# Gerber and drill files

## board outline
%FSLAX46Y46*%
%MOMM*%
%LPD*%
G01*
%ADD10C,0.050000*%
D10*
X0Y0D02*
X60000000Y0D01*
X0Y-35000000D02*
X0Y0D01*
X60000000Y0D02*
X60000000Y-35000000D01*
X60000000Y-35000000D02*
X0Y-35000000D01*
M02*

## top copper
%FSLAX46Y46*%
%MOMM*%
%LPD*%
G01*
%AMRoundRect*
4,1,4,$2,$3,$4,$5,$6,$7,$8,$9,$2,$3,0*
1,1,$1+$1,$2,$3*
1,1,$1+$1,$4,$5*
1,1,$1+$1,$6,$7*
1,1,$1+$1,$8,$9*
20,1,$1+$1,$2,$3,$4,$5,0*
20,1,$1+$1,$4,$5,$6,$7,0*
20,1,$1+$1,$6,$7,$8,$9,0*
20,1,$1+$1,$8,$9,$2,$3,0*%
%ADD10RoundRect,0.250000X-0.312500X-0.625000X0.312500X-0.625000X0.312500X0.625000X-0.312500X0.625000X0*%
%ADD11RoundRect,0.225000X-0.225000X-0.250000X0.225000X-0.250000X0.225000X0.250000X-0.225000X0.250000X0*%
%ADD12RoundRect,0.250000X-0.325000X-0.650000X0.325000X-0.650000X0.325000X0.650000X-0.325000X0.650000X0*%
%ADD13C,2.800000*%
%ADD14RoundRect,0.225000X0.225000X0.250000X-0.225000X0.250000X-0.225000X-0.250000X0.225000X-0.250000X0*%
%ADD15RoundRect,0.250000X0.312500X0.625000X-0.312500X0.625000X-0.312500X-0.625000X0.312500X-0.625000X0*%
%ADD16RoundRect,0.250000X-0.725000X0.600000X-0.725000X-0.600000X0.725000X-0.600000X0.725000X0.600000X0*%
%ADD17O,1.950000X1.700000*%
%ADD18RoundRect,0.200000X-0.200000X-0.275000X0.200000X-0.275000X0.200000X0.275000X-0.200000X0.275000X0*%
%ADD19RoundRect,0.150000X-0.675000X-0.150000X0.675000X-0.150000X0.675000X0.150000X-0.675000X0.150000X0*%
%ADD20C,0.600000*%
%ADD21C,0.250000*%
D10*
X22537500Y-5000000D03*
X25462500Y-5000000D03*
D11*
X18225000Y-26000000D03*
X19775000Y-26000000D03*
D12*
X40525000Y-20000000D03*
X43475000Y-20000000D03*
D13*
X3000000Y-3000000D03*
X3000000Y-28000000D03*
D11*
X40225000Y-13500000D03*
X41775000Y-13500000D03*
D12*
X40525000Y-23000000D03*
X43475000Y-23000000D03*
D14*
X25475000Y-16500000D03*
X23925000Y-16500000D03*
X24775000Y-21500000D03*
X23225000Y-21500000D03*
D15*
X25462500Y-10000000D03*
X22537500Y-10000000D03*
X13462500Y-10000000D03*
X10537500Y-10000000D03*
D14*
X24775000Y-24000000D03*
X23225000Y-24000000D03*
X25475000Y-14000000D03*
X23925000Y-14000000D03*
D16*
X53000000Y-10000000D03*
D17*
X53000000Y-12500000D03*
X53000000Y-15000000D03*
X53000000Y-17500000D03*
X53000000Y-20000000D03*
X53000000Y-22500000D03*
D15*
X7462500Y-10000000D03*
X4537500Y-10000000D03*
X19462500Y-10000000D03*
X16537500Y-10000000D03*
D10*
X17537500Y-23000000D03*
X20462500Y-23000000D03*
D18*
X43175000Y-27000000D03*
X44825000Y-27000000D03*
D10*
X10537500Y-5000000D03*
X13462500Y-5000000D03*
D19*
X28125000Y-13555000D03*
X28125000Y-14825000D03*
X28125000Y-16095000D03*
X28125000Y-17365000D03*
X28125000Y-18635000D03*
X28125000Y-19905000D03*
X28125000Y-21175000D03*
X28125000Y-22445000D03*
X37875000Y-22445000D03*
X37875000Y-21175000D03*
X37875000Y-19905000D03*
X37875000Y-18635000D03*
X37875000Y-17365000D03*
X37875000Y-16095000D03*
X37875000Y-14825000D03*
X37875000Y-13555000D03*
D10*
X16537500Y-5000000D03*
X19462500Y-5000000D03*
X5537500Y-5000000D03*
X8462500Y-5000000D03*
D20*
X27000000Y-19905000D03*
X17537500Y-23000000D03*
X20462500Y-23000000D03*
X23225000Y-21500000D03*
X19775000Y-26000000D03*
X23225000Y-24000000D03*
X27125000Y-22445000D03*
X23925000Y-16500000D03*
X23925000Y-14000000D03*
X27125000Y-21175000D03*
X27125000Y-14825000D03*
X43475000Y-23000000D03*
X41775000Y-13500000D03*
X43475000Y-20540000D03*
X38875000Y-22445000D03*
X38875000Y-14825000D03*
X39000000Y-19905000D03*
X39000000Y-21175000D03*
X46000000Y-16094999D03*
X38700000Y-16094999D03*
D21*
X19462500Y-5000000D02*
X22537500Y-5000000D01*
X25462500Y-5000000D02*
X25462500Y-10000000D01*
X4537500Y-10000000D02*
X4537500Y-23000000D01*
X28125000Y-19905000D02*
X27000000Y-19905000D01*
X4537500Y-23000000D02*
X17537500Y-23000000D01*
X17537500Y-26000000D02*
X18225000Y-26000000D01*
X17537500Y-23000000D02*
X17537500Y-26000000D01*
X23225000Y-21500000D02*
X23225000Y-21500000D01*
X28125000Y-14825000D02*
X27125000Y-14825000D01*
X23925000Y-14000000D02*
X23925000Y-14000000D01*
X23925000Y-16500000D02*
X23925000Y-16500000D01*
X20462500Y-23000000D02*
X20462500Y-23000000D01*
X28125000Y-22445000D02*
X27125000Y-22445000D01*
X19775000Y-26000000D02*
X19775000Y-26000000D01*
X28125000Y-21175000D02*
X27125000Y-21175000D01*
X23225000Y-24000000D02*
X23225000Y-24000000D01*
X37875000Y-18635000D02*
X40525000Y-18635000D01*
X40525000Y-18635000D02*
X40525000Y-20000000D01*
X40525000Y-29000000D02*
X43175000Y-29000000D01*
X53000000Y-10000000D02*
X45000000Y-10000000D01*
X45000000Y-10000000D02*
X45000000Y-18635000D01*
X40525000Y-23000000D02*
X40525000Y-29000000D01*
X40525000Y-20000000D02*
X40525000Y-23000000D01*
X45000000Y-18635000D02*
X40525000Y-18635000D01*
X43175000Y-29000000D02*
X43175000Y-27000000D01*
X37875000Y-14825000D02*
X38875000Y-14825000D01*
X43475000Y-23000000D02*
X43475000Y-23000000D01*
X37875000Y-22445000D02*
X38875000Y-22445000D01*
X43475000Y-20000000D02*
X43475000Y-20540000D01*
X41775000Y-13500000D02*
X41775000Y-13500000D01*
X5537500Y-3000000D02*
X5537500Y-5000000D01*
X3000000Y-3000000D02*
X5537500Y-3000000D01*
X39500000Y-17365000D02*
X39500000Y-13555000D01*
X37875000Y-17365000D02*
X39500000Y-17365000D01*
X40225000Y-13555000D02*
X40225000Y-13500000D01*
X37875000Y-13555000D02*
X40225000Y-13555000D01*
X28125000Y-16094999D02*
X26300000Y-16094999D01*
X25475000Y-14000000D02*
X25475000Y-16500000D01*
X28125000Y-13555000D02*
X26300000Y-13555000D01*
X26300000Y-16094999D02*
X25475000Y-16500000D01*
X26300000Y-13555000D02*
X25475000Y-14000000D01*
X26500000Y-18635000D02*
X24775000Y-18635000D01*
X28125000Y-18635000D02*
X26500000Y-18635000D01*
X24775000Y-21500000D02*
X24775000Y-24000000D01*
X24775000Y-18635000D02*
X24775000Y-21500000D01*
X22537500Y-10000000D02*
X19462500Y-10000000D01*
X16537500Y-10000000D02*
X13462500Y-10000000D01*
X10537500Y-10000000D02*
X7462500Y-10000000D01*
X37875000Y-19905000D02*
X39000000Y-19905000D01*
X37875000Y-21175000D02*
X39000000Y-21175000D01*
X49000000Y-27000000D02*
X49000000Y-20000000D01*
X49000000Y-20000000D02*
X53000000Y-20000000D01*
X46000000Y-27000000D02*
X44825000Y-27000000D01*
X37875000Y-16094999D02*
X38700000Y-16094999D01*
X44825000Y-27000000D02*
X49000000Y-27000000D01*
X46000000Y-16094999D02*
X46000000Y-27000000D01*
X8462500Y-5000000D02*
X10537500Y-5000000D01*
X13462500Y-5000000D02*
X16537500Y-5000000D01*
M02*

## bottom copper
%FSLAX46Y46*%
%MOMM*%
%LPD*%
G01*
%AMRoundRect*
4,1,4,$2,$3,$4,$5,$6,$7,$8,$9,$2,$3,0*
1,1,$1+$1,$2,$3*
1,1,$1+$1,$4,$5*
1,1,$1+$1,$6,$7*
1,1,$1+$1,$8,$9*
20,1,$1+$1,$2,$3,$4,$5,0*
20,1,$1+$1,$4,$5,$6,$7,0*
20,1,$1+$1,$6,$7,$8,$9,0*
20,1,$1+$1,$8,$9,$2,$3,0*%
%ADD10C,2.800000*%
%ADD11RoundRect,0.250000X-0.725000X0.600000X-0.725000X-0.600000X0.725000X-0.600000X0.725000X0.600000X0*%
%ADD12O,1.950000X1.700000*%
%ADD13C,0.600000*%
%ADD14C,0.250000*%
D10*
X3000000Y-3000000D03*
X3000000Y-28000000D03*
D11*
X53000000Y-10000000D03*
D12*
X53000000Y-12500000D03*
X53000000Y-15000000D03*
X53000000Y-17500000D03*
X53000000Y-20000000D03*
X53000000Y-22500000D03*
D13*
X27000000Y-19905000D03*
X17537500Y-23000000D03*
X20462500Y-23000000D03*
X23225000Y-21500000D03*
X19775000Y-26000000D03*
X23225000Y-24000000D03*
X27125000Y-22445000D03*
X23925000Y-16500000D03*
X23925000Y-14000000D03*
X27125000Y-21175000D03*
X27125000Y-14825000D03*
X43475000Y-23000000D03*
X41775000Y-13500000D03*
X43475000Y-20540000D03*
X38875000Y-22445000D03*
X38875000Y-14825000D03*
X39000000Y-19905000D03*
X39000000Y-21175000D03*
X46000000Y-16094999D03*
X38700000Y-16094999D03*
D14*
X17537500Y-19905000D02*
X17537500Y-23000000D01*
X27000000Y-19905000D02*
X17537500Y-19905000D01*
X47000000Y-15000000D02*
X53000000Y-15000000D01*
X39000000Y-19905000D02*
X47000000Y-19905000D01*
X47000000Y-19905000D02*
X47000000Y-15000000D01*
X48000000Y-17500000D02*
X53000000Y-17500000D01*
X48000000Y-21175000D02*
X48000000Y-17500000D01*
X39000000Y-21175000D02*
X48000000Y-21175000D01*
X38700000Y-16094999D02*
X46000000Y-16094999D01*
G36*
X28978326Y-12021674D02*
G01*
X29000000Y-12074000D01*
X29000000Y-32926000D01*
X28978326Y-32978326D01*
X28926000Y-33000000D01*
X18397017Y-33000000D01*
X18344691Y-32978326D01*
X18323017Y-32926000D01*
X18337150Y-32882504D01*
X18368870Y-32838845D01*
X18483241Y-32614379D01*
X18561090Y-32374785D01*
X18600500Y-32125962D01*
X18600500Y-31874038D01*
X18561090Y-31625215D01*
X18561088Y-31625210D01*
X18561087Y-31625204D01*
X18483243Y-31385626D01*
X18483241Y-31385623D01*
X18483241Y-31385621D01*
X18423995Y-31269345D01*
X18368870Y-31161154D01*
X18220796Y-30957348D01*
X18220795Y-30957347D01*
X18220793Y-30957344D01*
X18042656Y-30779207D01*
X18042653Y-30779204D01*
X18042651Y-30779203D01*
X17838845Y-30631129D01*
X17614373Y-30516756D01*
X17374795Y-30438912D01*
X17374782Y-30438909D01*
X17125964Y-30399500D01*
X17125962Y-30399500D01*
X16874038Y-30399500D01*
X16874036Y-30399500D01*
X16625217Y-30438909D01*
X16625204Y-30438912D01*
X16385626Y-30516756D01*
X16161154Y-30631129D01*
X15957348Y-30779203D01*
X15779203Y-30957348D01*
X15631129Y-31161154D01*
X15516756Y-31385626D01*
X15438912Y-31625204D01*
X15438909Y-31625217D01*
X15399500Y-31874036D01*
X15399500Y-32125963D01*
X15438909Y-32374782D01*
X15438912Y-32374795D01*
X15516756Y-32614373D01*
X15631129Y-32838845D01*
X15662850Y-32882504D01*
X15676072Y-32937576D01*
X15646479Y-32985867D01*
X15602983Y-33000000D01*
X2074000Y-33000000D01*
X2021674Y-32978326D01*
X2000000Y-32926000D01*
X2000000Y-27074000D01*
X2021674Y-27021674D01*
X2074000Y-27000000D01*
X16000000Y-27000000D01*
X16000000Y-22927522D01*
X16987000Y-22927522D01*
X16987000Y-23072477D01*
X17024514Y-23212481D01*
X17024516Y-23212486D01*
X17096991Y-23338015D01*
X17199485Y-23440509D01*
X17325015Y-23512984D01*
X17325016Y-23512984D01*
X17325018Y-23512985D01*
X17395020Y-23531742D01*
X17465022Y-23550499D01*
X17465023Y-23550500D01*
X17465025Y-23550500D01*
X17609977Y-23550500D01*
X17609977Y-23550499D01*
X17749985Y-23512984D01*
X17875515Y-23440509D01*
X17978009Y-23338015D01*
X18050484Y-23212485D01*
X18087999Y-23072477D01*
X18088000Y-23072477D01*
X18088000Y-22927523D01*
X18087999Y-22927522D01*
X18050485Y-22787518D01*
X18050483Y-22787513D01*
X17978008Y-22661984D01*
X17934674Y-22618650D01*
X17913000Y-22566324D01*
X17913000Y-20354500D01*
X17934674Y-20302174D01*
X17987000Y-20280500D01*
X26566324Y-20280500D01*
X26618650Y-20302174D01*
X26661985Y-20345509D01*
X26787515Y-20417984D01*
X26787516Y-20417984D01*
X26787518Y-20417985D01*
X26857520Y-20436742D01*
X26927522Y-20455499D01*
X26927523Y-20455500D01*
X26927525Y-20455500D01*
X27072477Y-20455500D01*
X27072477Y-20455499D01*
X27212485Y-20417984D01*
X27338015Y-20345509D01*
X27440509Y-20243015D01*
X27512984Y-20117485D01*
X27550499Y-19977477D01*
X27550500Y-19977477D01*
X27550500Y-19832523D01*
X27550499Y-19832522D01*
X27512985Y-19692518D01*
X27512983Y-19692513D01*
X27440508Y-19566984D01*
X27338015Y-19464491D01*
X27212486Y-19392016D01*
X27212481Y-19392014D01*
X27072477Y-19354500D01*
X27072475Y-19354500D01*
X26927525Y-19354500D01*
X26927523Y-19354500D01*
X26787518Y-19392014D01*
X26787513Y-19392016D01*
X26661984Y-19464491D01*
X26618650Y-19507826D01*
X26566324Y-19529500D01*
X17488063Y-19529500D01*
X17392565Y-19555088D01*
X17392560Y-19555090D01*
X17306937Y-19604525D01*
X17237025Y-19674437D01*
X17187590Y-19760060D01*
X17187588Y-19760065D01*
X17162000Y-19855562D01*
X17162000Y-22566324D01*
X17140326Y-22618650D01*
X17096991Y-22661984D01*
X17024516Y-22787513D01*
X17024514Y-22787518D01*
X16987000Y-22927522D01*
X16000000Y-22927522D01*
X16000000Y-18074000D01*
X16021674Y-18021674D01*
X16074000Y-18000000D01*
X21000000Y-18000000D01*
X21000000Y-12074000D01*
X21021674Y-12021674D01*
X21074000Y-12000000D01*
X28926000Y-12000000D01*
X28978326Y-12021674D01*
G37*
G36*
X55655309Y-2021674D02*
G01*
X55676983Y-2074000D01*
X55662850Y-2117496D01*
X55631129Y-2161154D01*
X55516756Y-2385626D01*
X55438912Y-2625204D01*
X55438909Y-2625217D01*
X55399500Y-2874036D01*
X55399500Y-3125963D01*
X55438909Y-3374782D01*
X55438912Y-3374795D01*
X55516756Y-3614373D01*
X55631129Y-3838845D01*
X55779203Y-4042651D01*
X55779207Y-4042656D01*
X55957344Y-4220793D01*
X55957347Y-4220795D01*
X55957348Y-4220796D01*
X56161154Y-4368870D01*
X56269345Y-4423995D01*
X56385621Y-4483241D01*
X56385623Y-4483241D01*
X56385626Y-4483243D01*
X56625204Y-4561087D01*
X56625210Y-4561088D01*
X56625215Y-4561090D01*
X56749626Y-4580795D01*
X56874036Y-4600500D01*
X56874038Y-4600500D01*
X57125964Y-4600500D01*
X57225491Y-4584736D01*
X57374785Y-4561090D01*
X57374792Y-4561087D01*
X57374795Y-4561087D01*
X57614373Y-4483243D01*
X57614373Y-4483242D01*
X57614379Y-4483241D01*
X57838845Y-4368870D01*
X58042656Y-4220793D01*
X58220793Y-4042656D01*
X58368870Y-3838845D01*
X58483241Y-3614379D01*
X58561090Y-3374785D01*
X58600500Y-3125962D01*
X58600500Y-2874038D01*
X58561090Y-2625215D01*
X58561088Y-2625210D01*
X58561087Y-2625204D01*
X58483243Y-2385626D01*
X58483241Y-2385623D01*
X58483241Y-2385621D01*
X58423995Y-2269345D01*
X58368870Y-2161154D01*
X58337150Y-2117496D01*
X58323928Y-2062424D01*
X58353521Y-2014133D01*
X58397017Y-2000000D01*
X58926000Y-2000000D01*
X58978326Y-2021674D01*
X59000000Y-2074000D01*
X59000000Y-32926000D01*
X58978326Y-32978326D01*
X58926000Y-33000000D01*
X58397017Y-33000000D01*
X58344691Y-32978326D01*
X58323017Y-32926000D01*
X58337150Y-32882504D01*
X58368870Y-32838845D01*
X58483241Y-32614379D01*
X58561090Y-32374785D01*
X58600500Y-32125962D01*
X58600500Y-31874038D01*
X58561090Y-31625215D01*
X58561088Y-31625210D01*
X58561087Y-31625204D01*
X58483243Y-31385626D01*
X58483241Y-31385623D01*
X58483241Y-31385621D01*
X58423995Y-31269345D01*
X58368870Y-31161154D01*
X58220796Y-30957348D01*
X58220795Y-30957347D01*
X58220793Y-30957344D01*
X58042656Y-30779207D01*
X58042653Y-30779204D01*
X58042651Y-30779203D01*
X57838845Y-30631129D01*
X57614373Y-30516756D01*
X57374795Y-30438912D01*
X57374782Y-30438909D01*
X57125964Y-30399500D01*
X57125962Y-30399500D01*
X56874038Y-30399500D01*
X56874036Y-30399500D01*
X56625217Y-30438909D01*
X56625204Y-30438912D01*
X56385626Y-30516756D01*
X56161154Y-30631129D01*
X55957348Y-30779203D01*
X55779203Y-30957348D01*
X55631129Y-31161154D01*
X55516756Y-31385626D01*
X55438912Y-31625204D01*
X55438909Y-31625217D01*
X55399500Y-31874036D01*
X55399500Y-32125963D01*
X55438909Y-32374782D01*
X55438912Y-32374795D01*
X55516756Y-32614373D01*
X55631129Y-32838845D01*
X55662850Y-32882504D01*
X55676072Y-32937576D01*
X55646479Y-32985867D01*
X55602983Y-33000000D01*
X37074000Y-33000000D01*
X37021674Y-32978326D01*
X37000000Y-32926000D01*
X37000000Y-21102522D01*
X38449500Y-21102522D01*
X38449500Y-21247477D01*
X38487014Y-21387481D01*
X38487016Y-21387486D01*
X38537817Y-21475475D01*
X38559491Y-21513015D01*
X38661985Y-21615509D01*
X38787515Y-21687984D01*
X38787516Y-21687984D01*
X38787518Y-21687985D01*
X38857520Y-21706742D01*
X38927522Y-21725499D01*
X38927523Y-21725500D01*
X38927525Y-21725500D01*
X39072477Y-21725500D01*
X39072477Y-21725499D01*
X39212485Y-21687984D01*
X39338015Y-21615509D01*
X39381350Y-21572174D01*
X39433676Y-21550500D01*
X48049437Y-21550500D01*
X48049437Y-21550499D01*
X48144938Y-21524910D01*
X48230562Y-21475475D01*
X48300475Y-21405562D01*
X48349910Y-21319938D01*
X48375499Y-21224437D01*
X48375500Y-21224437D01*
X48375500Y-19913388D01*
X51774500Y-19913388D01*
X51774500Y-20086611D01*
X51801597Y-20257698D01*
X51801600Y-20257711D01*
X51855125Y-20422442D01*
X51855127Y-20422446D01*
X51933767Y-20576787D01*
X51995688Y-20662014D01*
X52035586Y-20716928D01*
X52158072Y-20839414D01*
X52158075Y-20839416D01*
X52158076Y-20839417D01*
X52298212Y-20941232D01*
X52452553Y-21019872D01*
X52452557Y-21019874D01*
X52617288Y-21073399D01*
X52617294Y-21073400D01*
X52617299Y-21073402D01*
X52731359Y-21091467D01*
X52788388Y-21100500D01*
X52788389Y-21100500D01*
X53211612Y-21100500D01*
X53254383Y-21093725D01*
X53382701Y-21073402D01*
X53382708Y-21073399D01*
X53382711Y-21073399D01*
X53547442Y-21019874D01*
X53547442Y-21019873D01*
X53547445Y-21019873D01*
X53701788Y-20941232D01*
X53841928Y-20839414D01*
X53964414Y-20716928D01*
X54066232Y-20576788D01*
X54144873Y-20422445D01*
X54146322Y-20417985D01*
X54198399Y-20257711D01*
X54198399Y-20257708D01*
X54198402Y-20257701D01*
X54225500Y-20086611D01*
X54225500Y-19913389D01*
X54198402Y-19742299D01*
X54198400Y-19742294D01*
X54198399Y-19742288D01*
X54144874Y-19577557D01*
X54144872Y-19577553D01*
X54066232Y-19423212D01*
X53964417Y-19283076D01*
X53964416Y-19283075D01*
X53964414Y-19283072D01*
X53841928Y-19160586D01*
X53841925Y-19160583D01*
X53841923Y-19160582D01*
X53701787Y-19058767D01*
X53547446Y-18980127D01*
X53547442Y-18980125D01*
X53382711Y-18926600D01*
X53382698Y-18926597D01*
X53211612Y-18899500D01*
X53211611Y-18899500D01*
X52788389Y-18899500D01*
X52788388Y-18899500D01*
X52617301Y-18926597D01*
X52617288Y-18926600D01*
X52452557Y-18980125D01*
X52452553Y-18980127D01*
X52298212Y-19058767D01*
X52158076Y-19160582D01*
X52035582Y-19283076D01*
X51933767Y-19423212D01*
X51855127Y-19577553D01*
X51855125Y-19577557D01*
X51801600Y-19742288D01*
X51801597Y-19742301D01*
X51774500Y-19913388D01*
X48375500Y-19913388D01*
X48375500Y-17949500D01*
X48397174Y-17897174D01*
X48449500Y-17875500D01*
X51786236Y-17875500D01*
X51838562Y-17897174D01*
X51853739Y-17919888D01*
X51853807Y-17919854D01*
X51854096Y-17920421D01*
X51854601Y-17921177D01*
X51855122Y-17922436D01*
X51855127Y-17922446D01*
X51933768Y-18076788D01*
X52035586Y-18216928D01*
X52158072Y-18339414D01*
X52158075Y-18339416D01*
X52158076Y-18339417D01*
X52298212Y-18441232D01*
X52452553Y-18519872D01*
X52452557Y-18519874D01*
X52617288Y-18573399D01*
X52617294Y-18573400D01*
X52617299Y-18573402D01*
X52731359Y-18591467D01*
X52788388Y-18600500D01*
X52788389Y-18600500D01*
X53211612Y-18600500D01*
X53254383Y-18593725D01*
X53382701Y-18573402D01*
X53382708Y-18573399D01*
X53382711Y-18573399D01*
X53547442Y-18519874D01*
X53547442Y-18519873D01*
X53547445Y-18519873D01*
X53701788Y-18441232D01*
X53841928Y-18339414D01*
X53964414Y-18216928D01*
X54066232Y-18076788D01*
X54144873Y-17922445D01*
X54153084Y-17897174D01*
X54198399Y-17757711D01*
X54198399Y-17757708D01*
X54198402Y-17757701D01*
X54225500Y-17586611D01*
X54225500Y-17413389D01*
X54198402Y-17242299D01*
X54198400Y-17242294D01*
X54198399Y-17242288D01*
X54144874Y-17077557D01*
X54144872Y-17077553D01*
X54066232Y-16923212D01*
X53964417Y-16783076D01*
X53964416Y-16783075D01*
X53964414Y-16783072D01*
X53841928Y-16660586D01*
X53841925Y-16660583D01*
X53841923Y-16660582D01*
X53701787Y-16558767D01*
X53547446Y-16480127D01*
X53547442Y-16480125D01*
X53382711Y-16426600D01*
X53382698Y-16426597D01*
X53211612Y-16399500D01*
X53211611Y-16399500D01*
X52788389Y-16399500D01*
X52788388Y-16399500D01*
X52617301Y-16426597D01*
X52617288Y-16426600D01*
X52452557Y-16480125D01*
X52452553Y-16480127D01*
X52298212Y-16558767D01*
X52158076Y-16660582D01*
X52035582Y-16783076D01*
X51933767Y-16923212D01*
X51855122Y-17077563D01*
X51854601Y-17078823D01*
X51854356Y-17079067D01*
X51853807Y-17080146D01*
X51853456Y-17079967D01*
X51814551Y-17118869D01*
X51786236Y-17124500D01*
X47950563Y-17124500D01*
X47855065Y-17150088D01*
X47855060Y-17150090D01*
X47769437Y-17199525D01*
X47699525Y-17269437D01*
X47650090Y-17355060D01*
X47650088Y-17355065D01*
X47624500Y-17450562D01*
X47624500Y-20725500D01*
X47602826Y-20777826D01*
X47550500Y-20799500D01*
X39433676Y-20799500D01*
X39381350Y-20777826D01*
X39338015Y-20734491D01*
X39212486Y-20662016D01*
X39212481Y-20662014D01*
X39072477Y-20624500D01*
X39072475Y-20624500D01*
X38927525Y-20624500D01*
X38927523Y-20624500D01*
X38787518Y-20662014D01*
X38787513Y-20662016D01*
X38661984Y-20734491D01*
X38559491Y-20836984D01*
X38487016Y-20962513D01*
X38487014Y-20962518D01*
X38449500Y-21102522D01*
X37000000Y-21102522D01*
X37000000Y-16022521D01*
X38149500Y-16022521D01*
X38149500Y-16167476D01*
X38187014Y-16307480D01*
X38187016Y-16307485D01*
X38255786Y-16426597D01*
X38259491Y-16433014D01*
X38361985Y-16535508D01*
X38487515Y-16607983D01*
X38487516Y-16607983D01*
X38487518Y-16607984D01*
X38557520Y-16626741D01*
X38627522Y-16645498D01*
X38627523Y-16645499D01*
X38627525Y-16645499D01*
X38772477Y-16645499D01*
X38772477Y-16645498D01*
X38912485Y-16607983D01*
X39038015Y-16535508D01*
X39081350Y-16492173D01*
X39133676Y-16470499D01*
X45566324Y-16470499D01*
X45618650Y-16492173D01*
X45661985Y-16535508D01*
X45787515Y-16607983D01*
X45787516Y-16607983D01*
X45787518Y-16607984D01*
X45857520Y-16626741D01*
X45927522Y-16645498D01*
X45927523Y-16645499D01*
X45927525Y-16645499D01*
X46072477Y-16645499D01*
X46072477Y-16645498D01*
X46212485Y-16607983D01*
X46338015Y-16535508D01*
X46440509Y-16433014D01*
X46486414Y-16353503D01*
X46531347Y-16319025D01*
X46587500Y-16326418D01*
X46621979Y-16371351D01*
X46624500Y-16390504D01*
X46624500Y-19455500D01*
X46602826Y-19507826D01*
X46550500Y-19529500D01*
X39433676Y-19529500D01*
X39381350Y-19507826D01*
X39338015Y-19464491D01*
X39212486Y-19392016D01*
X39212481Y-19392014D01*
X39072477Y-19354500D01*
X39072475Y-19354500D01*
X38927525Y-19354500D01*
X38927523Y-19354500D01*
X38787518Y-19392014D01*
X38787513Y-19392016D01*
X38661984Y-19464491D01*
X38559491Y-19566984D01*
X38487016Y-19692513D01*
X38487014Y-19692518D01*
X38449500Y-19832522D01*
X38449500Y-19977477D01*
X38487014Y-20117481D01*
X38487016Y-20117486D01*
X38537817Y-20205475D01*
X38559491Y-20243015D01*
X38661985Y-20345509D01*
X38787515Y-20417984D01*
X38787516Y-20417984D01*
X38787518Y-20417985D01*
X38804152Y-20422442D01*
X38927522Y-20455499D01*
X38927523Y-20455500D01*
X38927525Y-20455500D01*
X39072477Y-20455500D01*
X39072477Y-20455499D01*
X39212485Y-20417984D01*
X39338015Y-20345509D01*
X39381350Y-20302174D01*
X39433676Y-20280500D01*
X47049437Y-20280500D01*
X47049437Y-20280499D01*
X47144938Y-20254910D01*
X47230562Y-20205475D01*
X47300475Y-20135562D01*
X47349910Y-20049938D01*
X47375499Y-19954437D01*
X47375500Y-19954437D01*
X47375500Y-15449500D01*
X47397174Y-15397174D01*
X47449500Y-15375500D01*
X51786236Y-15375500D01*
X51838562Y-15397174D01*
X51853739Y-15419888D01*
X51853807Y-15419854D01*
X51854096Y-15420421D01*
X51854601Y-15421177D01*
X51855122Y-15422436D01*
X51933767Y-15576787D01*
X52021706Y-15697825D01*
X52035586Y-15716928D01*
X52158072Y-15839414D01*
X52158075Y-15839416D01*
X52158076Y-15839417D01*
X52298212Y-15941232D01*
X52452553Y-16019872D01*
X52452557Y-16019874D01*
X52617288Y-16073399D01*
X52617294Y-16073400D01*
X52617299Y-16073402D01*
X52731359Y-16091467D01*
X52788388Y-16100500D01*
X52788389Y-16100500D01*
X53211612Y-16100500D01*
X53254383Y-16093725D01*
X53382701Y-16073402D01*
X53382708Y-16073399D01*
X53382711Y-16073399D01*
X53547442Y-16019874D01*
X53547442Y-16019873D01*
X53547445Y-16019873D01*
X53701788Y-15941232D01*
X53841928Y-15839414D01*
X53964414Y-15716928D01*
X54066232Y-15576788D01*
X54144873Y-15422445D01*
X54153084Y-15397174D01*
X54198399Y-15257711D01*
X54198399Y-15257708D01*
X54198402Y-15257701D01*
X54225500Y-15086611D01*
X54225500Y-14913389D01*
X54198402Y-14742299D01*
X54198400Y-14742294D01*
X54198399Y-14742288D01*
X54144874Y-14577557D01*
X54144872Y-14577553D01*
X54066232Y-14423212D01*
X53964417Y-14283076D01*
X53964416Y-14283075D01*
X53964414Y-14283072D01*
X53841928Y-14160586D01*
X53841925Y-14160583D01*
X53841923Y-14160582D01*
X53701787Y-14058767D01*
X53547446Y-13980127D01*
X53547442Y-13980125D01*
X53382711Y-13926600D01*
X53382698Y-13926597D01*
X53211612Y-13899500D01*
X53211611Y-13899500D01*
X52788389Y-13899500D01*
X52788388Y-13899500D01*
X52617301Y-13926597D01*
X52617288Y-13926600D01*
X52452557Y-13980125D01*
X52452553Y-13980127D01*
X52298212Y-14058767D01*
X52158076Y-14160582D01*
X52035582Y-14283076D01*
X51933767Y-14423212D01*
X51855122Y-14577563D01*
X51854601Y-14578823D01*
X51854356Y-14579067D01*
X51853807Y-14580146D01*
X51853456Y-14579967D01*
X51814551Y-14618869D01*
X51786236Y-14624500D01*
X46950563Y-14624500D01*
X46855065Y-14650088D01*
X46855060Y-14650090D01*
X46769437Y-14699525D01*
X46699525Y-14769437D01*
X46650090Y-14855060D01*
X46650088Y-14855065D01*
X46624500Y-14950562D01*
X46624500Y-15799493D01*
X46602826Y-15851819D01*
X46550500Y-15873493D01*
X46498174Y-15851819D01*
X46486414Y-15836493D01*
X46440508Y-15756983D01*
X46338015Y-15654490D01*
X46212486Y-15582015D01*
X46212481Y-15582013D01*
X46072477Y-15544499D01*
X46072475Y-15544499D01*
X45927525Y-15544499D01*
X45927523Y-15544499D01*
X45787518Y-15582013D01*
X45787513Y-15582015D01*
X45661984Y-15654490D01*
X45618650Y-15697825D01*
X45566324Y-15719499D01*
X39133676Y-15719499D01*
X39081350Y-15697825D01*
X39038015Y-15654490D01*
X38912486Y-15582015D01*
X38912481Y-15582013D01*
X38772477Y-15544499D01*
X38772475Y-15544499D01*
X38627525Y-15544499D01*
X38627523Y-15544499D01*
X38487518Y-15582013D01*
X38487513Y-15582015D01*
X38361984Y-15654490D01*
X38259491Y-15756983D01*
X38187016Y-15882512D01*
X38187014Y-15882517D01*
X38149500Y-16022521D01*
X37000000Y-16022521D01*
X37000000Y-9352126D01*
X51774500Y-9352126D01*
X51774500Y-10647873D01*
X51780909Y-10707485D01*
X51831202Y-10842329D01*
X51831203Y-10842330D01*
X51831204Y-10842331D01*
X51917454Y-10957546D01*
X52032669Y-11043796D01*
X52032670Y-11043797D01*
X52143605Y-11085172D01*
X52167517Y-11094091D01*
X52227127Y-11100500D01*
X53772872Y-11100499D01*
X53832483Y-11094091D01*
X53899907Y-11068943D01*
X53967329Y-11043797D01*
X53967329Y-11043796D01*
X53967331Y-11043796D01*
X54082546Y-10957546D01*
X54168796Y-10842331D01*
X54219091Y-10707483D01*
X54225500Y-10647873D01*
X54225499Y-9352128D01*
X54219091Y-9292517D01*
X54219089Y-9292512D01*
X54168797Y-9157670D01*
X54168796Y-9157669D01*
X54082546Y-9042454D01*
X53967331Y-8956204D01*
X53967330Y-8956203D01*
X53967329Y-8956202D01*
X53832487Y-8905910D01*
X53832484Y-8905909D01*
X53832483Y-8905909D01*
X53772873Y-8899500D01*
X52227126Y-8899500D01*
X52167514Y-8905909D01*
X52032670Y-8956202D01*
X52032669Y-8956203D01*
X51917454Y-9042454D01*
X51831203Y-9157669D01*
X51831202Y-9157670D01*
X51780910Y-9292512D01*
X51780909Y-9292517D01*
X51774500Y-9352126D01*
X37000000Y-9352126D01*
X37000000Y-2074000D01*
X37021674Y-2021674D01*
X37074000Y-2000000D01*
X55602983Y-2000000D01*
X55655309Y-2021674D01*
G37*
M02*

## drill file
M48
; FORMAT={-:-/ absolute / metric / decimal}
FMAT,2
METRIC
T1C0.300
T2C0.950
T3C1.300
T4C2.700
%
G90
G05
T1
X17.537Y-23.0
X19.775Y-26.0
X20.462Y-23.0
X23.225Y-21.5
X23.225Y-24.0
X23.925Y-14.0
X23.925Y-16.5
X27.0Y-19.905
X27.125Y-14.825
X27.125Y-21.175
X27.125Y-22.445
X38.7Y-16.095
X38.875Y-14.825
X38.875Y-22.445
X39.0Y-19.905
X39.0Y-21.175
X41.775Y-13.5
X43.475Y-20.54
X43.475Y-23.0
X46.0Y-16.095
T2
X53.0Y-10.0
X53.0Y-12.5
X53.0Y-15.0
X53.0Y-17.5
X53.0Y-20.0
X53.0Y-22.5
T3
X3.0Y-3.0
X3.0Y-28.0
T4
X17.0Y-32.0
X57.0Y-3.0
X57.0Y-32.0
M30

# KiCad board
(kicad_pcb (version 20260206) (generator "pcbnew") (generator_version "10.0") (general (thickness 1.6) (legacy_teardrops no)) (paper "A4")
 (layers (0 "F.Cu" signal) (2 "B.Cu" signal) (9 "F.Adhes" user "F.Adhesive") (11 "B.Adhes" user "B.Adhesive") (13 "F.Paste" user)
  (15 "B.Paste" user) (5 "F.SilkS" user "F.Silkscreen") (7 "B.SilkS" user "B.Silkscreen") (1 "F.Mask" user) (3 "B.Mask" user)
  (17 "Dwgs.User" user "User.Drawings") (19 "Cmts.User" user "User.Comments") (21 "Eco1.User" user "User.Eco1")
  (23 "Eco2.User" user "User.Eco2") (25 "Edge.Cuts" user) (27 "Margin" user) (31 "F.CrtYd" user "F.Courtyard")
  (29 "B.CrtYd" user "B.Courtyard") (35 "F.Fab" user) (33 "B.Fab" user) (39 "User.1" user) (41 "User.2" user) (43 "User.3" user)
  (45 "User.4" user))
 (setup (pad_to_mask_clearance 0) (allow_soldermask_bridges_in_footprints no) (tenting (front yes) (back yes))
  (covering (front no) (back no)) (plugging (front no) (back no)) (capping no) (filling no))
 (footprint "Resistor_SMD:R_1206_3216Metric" (layer "F.Cu") (at 24 5)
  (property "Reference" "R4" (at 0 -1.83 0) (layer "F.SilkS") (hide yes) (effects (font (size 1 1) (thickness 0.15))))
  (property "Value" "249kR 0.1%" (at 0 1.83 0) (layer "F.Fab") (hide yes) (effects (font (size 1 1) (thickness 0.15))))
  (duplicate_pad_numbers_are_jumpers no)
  (pad "1" smd roundrect (at -1.4625 0) (size 1.125 1.75) (layers "F.Cu" "F.Mask" "F.Paste") (roundrect_rratio 0.222222) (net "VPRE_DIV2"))
  (pad "2" smd roundrect (at 1.4625 0) (size 1.125 1.75) (layers "F.Cu" "F.Mask" "F.Paste") (roundrect_rratio 0.222222) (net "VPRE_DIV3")))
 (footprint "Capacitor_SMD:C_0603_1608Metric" (layer "F.Cu") (at 19 26)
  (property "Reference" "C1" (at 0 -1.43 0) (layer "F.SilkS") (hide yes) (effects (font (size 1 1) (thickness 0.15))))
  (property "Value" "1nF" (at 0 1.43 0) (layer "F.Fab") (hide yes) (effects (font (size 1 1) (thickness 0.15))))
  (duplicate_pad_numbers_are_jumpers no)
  (pad "1" smd roundrect (at -0.775 0) (size 0.9 0.95) (layers "F.Cu" "F.Mask" "F.Paste") (roundrect_rratio 0.25) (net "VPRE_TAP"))
  (pad "2" smd roundrect (at 0.775 0) (size 0.9 0.95) (layers "F.Cu" "F.Mask" "F.Paste") (roundrect_rratio 0.25) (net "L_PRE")))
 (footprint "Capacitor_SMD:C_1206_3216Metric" (layer "F.Cu") (at 42 20)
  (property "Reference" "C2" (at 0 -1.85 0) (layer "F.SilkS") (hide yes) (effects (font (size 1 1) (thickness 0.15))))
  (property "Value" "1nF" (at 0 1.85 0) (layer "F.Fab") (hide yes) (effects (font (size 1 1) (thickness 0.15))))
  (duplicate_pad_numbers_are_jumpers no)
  (pad "1" smd roundrect (at -1.475 0) (size 1.15 1.8) (layers "F.Cu" "F.Mask" "F.Paste") (roundrect_rratio 0.217391) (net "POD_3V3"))
  (pad "2" smd roundrect (at 1.475 0) (size 1.15 1.8) (layers "F.Cu" "F.Mask" "F.Paste") (roundrect_rratio 0.217391) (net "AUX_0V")))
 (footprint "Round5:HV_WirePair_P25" (layer "F.Cu") (at 3 3)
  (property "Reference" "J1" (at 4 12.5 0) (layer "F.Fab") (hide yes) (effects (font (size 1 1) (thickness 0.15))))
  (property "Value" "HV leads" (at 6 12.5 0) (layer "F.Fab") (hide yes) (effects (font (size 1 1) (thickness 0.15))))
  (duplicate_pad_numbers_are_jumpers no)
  (pad "1" thru_hole circle (at 0 0) (size 2.8 2.8) (drill 1.3) (layers "*.Cu" "*.Mask") (remove_unused_layers no) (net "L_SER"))
  (pad "2" thru_hole circle (at 0 25) (size 2.8 2.8) (drill 1.3) (layers "*.Cu" "*.Mask") (remove_unused_layers no) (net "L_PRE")))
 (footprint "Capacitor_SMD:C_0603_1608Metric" (layer "F.Cu") (at 41 13.5)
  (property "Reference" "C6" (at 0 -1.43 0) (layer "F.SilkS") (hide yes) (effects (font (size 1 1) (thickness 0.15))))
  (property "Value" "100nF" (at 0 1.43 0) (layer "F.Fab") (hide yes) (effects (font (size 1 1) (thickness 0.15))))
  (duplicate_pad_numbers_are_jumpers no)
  (pad "1" smd roundrect (at -0.775 0) (size 0.9 0.95) (layers "F.Cu" "F.Mask" "F.Paste") (roundrect_rratio 0.25) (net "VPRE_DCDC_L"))
  (pad "2" smd roundrect (at 0.775 0) (size 0.9 0.95) (layers "F.Cu" "F.Mask" "F.Paste") (roundrect_rratio 0.25) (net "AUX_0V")))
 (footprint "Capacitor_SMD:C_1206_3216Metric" (layer "F.Cu") (at 42 23)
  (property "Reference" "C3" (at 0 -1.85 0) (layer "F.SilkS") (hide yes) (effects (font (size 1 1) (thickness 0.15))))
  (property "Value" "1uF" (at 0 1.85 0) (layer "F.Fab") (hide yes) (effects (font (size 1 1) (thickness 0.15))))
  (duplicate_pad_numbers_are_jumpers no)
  (pad "1" smd roundrect (at -1.475 0) (size 1.15 1.8) (layers "F.Cu" "F.Mask" "F.Paste") (roundrect_rratio 0.217391) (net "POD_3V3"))
  (pad "2" smd roundrect (at 1.475 0) (size 1.15 1.8) (layers "F.Cu" "F.Mask" "F.Paste") (roundrect_rratio 0.217391) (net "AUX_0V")))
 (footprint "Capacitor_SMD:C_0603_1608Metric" (layer "F.Cu") (at 24.7 16.5 180)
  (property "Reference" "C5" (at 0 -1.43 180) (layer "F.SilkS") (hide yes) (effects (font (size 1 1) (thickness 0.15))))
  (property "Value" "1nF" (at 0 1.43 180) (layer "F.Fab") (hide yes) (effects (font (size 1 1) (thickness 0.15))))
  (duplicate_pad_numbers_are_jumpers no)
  (pad "1" smd roundrect (at -0.775 0 180) (size 0.9 0.95) (layers "F.Cu" "F.Mask" "F.Paste") (roundrect_rratio 0.25) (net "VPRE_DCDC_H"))
  (pad "2" smd roundrect (at 0.775 0 180) (size 0.9 0.95) (layers "F.Cu" "F.Mask" "F.Paste") (roundrect_rratio 0.25) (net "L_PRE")))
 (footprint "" (layer "F.Cu") (at 57 3)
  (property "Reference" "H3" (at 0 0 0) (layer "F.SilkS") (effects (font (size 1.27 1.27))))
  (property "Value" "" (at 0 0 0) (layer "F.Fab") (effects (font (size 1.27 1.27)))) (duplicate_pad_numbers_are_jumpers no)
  (pad "" np_thru_hole circle (at 0 0) (size 2.7 2.7) (drill 2.7) (layers "*.Cu")))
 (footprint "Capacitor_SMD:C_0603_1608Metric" (layer "F.Cu") (at 24 21.5 180)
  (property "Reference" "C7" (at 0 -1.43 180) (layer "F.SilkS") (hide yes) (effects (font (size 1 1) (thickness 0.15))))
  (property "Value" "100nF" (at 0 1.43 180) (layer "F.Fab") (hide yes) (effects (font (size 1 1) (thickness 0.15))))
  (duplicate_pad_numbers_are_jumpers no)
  (pad "1" smd roundrect (at -0.775 0 180) (size 0.9 0.95) (layers "F.Cu" "F.Mask" "F.Paste") (roundrect_rratio 0.25) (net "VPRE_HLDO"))
  (pad "2" smd roundrect (at 0.775 0 180) (size 0.9 0.95) (layers "F.Cu" "F.Mask" "F.Paste") (roundrect_rratio 0.25) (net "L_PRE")))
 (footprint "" (layer "F.Cu") (at 57 32)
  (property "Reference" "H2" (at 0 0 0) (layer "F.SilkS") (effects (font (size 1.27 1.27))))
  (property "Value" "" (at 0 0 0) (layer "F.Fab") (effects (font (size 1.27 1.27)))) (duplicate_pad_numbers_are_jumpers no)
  (pad "" np_thru_hole circle (at 0 0) (size 2.7 2.7) (drill 2.7) (layers "*.Cu")))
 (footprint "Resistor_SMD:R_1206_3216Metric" (layer "F.Cu") (at 24 10 180)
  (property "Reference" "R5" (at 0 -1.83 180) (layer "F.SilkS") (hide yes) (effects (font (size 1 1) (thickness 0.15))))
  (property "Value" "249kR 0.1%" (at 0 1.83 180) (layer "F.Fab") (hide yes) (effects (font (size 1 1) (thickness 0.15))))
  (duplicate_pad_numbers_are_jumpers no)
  (pad "1" smd roundrect (at -1.4625 0 180) (size 1.125 1.75) (layers "F.Cu" "F.Mask" "F.Paste") (roundrect_rratio 0.222222)
   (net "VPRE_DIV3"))
  (pad "2" smd roundrect (at 1.4625 0 180) (size 1.125 1.75) (layers "F.Cu" "F.Mask" "F.Paste") (roundrect_rratio 0.222222)
   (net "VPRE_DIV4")))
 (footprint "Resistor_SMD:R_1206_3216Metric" (layer "F.Cu") (at 12 10 180)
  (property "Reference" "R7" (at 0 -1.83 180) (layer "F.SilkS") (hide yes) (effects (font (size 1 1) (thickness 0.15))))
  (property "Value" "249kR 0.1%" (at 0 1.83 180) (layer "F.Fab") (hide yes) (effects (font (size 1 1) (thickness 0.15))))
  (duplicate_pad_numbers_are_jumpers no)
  (pad "1" smd roundrect (at -1.4625 0 180) (size 1.125 1.75) (layers "F.Cu" "F.Mask" "F.Paste") (roundrect_rratio 0.222222)
   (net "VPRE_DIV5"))
  (pad "2" smd roundrect (at 1.4625 0 180) (size 1.125 1.75) (layers "F.Cu" "F.Mask" "F.Paste") (roundrect_rratio 0.222222)
   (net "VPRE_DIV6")))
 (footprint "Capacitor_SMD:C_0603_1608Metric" (layer "F.Cu") (at 24 24 180)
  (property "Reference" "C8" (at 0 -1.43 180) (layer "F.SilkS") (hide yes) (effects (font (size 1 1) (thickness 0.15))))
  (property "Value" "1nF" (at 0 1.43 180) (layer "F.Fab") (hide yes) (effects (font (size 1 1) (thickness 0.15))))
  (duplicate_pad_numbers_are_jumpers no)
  (pad "1" smd roundrect (at -0.775 0 180) (size 0.9 0.95) (layers "F.Cu" "F.Mask" "F.Paste") (roundrect_rratio 0.25) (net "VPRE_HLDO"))
  (pad "2" smd roundrect (at 0.775 0 180) (size 0.9 0.95) (layers "F.Cu" "F.Mask" "F.Paste") (roundrect_rratio 0.25) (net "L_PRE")))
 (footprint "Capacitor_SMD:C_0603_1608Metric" (layer "F.Cu") (at 24.7 14 180)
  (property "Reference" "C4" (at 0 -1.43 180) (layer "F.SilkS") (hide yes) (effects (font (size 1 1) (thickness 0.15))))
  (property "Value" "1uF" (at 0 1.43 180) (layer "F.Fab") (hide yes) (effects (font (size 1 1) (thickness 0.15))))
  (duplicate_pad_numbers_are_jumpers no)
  (pad "1" smd roundrect (at -0.775 0 180) (size 0.9 0.95) (layers "F.Cu" "F.Mask" "F.Paste") (roundrect_rratio 0.25) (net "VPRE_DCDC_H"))
  (pad "2" smd roundrect (at 0.775 0 180) (size 0.9 0.95) (layers "F.Cu" "F.Mask" "F.Paste") (roundrect_rratio 0.25) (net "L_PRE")))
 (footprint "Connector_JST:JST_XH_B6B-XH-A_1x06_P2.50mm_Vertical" (layer "F.Cu") (at 53 10 -90)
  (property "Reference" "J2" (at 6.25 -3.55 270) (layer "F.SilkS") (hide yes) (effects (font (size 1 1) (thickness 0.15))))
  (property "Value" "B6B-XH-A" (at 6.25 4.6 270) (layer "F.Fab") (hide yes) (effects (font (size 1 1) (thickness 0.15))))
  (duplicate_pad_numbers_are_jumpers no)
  (pad "1" thru_hole roundrect (at 0 0 270) (size 1.7 1.95) (drill 0.95) (layers "*.Cu" "*.Mask") (remove_unused_layers no)
   (roundrect_rratio 0.147059) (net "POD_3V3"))
  (pad "2" thru_hole oval (at 2.5 0 270) (size 1.7 1.95) (drill 0.95) (layers "*.Cu" "*.Mask") (remove_unused_layers no) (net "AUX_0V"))
  (pad "3" thru_hole oval (at 5 0 270) (size 1.7 1.95) (drill 0.95) (layers "*.Cu" "*.Mask") (remove_unused_layers no) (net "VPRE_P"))
  (pad "4" thru_hole oval (at 7.5 0 270) (size 1.7 1.95) (drill 0.95) (layers "*.Cu" "*.Mask") (remove_unused_layers no) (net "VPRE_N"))
  (pad "5" thru_hole oval (at 10 0 270) (size 1.7 1.95) (drill 0.95) (layers "*.Cu" "*.Mask") (remove_unused_layers no) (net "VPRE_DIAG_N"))
  (pad "6" thru_hole oval (at 12.5 0 270) (size 1.7 1.95) (drill 0.95) (layers "*.Cu" "*.Mask") (remove_unused_layers no) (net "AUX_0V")))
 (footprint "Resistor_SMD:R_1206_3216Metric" (layer "F.Cu") (at 6 10 180)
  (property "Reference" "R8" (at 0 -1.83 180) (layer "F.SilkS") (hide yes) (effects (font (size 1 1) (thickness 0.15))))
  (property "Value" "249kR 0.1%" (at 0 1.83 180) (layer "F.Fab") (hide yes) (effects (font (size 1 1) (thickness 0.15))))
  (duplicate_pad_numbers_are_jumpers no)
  (pad "1" smd roundrect (at -1.4625 0 180) (size 1.125 1.75) (layers "F.Cu" "F.Mask" "F.Paste") (roundrect_rratio 0.222222)
   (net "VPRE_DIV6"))
  (pad "2" smd roundrect (at 1.4625 0 180) (size 1.125 1.75) (layers "F.Cu" "F.Mask" "F.Paste") (roundrect_rratio 0.222222) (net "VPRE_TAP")))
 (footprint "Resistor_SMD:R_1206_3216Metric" (layer "F.Cu") (at 18 10 180)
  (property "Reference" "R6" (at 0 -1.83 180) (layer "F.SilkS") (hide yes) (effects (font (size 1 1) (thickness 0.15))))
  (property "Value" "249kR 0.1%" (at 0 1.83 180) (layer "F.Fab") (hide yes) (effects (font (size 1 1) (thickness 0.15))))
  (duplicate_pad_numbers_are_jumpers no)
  (pad "1" smd roundrect (at -1.4625 0 180) (size 1.125 1.75) (layers "F.Cu" "F.Mask" "F.Paste") (roundrect_rratio 0.222222)
   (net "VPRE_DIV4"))
  (pad "2" smd roundrect (at 1.4625 0 180) (size 1.125 1.75) (layers "F.Cu" "F.Mask" "F.Paste") (roundrect_rratio 0.222222)
   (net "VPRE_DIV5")))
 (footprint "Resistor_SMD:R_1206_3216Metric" (layer "F.Cu") (at 19 23)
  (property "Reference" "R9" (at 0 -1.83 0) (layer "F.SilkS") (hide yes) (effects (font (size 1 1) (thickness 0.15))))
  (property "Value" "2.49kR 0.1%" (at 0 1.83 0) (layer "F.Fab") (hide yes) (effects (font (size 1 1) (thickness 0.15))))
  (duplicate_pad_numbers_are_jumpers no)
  (pad "1" smd roundrect (at -1.4625 0) (size 1.125 1.75) (layers "F.Cu" "F.Mask" "F.Paste") (roundrect_rratio 0.222222) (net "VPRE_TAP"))
  (pad "2" smd roundrect (at 1.4625 0) (size 1.125 1.75) (layers "F.Cu" "F.Mask" "F.Paste") (roundrect_rratio 0.222222) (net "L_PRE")))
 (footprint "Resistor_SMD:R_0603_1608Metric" (layer "F.Cu") (at 44 27)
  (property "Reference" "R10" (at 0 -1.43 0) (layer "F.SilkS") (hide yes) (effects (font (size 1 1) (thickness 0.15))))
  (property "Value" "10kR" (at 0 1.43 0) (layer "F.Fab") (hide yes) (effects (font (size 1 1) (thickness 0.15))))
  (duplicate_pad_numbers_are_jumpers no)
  (pad "1" smd roundrect (at -0.825 0) (size 0.8 0.95) (layers "F.Cu" "F.Mask" "F.Paste") (roundrect_rratio 0.25) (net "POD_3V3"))
  (pad "2" smd roundrect (at 0.825 0) (size 0.8 0.95) (layers "F.Cu" "F.Mask" "F.Paste") (roundrect_rratio 0.25) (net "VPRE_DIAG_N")))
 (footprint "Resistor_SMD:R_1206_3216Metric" (layer "F.Cu") (at 12 5)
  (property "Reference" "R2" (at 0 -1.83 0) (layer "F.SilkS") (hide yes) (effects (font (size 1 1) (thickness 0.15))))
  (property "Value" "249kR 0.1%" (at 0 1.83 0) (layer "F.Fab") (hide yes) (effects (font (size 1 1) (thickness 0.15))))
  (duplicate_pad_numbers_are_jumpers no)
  (pad "1" smd roundrect (at -1.4625 0) (size 1.125 1.75) (layers "F.Cu" "F.Mask" "F.Paste") (roundrect_rratio 0.222222) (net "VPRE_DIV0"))
  (pad "2" smd roundrect (at 1.4625 0) (size 1.125 1.75) (layers "F.Cu" "F.Mask" "F.Paste") (roundrect_rratio 0.222222) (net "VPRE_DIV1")))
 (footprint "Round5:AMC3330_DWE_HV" (layer "F.Cu") (at 33 18)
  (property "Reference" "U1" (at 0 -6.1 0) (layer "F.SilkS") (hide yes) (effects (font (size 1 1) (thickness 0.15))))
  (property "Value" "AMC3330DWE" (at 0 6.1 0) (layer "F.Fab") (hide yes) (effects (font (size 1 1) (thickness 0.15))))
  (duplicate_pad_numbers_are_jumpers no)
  (pad "1" smd roundrect (at -4.875 -4.445) (size 1.65 0.6) (layers "F.Cu" "F.Mask" "F.Paste") (roundrect_rratio 0.25) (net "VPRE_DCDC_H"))
  (pad "2" smd roundrect (at -4.875 -3.175) (size 1.65 0.6) (layers "F.Cu" "F.Mask" "F.Paste") (roundrect_rratio 0.25) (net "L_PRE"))
  (pad "3" smd roundrect (at -4.875 -1.905) (size 1.65 0.6) (layers "F.Cu" "F.Mask" "F.Paste") (roundrect_rratio 0.25) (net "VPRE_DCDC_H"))
  (pad "4" smd roundrect (at -4.875 -0.635) (size 1.65 0.6) (layers "F.Cu" "F.Mask" "F.Paste") (roundrect_rratio 0.25)
   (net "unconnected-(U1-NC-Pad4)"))
  (pad "5" smd roundrect (at -4.875 0.635) (size 1.65 0.6) (layers "F.Cu" "F.Mask" "F.Paste") (roundrect_rratio 0.25) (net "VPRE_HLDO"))
  (pad "6" smd roundrect (at -4.875 1.905) (size 1.65 0.6) (layers "F.Cu" "F.Mask" "F.Paste") (roundrect_rratio 0.25) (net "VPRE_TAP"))
  (pad "7" smd roundrect (at -4.875 3.175) (size 1.65 0.6) (layers "F.Cu" "F.Mask" "F.Paste") (roundrect_rratio 0.25) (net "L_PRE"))
  (pad "8" smd roundrect (at -4.875 4.445) (size 1.65 0.6) (layers "F.Cu" "F.Mask" "F.Paste") (roundrect_rratio 0.25) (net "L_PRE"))
  (pad "9" smd roundrect (at 4.875 4.445) (size 1.65 0.6) (layers "F.Cu" "F.Mask" "F.Paste") (roundrect_rratio 0.25) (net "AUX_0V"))
  (pad "10" smd roundrect (at 4.875 3.175) (size 1.65 0.6) (layers "F.Cu" "F.Mask" "F.Paste") (roundrect_rratio 0.25) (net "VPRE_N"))
  (pad "11" smd roundrect (at 4.875 1.905) (size 1.65 0.6) (layers "F.Cu" "F.Mask" "F.Paste") (roundrect_rratio 0.25) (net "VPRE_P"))
  (pad "12" smd roundrect (at 4.875 0.635) (size 1.65 0.6) (layers "F.Cu" "F.Mask" "F.Paste") (roundrect_rratio 0.25) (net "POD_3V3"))
  (pad "13" smd roundrect (at 4.875 -0.635) (size 1.65 0.6) (layers "F.Cu" "F.Mask" "F.Paste") (roundrect_rratio 0.25) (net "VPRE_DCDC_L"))
  (pad "14" smd roundrect (at 4.875 -1.905) (size 1.65 0.6) (layers "F.Cu" "F.Mask" "F.Paste") (roundrect_rratio 0.25) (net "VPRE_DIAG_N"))
  (pad "15" smd roundrect (at 4.875 -3.175) (size 1.65 0.6) (layers "F.Cu" "F.Mask" "F.Paste") (roundrect_rratio 0.25) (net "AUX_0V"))
  (pad "16" smd roundrect (at 4.875 -4.445) (size 1.65 0.6) (layers "F.Cu" "F.Mask" "F.Paste") (roundrect_rratio 0.25) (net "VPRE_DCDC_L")))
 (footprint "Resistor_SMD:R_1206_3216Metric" (layer "F.Cu") (at 18 5)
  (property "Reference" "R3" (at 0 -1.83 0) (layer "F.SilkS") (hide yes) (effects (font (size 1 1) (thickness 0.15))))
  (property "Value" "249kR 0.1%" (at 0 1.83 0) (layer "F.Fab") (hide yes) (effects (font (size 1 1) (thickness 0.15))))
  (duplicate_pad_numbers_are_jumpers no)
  (pad "1" smd roundrect (at -1.4625 0) (size 1.125 1.75) (layers "F.Cu" "F.Mask" "F.Paste") (roundrect_rratio 0.222222) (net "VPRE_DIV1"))
  (pad "2" smd roundrect (at 1.4625 0) (size 1.125 1.75) (layers "F.Cu" "F.Mask" "F.Paste") (roundrect_rratio 0.222222) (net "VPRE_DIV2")))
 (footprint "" (layer "F.Cu") (at 17 32)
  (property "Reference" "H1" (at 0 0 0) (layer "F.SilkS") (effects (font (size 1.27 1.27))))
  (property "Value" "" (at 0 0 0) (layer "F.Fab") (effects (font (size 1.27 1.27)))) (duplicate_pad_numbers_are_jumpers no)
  (pad "" np_thru_hole circle (at 0 0) (size 2.7 2.7) (drill 2.7) (layers "*.Cu")))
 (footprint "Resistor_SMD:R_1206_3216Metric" (layer "F.Cu") (at 7 5)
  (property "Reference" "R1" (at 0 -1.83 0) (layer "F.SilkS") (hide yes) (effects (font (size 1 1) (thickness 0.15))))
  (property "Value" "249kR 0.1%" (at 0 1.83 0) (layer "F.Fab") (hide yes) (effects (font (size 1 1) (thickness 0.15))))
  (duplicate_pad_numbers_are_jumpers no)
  (pad "1" smd roundrect (at -1.4625 0) (size 1.125 1.75) (layers "F.Cu" "F.Mask" "F.Paste") (roundrect_rratio 0.222222) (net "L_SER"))
  (pad "2" smd roundrect (at 1.4625 0) (size 1.125 1.75) (layers "F.Cu" "F.Mask" "F.Paste") (roundrect_rratio 0.222222) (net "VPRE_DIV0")))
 (gr_line (start 0 0) (end 60 0) (stroke (width 0.05) (type default)) (layer "Edge.Cuts"))
 (gr_line (start 0 35) (end 0 0) (stroke (width 0.05) (type default)) (layer "Edge.Cuts"))
 (gr_line (start 60 0) (end 60 35) (stroke (width 0.05) (type default)) (layer "Edge.Cuts"))
 (gr_line (start 60 35) (end 0 35) (stroke (width 0.05) (type default)) (layer "Edge.Cuts"))
 (segment (start 19.4625 5) (end 22.5375 5) (width 0.25) (layer "F.Cu") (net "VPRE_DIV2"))
 (segment (start 25.4625 5) (end 25.4625 10) (width 0.25) (layer "F.Cu") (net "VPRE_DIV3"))
 (segment (start 4.5375 10) (end 4.5375 23) (width 0.25) (layer "F.Cu") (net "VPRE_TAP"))
 (segment (start 28.125 19.905) (end 27 19.905) (width 0.25) (layer "F.Cu") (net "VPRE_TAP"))
 (segment (start 4.5375 23) (end 17.5375 23) (width 0.25) (layer "F.Cu") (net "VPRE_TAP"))
 (segment (start 17.5375 26) (end 18.225 26) (width 0.25) (layer "F.Cu") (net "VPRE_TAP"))
 (segment (start 17.5375 23) (end 17.5375 26) (width 0.25) (layer "F.Cu") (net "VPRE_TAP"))
 (via (at 27 19.905) (size 0.6) (drill 0.3) (layers "F.Cu" "B.Cu") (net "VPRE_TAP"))
 (via (at 17.5375 23) (size 0.6) (drill 0.3) (layers "F.Cu" "B.Cu") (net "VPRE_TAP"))
 (segment (start 17.5375 19.905) (end 17.5375 23) (width 0.25) (layer "B.Cu") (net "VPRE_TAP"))
 (segment (start 27 19.905) (end 17.5375 19.905) (width 0.25) (layer "B.Cu") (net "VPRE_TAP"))
 (segment (start 23.225 21.5) (end 23.225 21.5) (width 0.25) (layer "F.Cu") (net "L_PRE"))
 (segment (start 28.125 14.825) (end 27.125 14.825) (width 0.25) (layer "F.Cu") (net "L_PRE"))
 (segment (start 23.925 14) (end 23.925 14) (width 0.25) (layer "F.Cu") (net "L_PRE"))
 (segment (start 23.925 16.5) (end 23.925 16.5) (width 0.25) (layer "F.Cu") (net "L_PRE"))
 (segment (start 20.4625 23) (end 20.4625 23) (width 0.25) (layer "F.Cu") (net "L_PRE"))
 (segment (start 28.125 22.445) (end 27.125 22.445) (width 0.25) (layer "F.Cu") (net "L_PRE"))
 (segment (start 19.775 26) (end 19.775 26) (width 0.25) (layer "F.Cu") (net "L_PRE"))
 (segment (start 28.125 21.175) (end 27.125 21.175) (width 0.25) (layer "F.Cu") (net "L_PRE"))
 (segment (start 23.225 24) (end 23.225 24) (width 0.25) (layer "F.Cu") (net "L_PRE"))
 (via (at 20.4625 23) (size 0.6) (drill 0.3) (layers "F.Cu" "B.Cu") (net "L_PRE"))
 (via (at 23.225 21.5) (size 0.6) (drill 0.3) (layers "F.Cu" "B.Cu") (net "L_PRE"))
 (via (at 19.775 26) (size 0.6) (drill 0.3) (layers "F.Cu" "B.Cu") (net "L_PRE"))
 (via (at 23.225 24) (size 0.6) (drill 0.3) (layers "F.Cu" "B.Cu") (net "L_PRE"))
 (via (at 27.125 22.445) (size 0.6) (drill 0.3) (layers "F.Cu" "B.Cu") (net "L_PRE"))
 (via (at 23.925 16.5) (size 0.6) (drill 0.3) (layers "F.Cu" "B.Cu") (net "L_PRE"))
 (via (at 23.925 14) (size 0.6) (drill 0.3) (layers "F.Cu" "B.Cu") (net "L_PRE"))
 (via (at 27.125 21.175) (size 0.6) (drill 0.3) (layers "F.Cu" "B.Cu") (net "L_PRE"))
 (via (at 27.125 14.825) (size 0.6) (drill 0.3) (layers "F.Cu" "B.Cu") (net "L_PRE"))
 (segment (start 37.875 18.635) (end 40.525 18.635) (width 0.25) (layer "F.Cu") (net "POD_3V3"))
 (segment (start 40.525 18.635) (end 40.525 20) (width 0.25) (layer "F.Cu") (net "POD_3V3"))
 (segment (start 40.525 29) (end 43.175 29) (width 0.25) (layer "F.Cu") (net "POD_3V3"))
 (segment (start 53 10) (end 45 10) (width 0.25) (layer "F.Cu") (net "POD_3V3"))
 (segment (start 45 10) (end 45 18.635) (width 0.25) (layer "F.Cu") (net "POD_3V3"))
 (segment (start 40.525 23) (end 40.525 29) (width 0.25) (layer "F.Cu") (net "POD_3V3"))
 (segment (start 40.525 20) (end 40.525 23) (width 0.25) (layer "F.Cu") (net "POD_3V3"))
 (segment (start 45 18.635) (end 40.525 18.635) (width 0.25) (layer "F.Cu") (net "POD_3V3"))
 (segment (start 43.175 29) (end 43.175 27) (width 0.25) (layer "F.Cu") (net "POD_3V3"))
 (segment (start 37.875 14.825) (end 38.875 14.825) (width 0.25) (layer "F.Cu") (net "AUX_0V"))
 (segment (start 43.475 23) (end 43.475 23) (width 0.25) (layer "F.Cu") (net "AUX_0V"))
 (segment (start 37.875 22.445) (end 38.875 22.445) (width 0.25) (layer "F.Cu") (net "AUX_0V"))
 (segment (start 43.475 20) (end 43.475 20.54) (width 0.25) (layer "F.Cu") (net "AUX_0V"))
 (segment (start 41.775 13.5) (end 41.775 13.5) (width 0.25) (layer "F.Cu") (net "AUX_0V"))
 (via (at 43.475 23) (size 0.6) (drill 0.3) (layers "F.Cu" "B.Cu") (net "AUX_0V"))
 (via (at 41.775 13.5) (size 0.6) (drill 0.3) (layers "F.Cu" "B.Cu") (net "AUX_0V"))
 (via (at 43.475 20.54) (size 0.6) (drill 0.3) (layers "F.Cu" "B.Cu") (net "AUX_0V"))
 (via (at 38.875 22.445) (size 0.6) (drill 0.3) (layers "F.Cu" "B.Cu") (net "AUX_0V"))
 (via (at 38.875 14.825) (size 0.6) (drill 0.3) (layers "F.Cu" "B.Cu") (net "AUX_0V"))
 (segment (start 5.5375 3) (end 5.5375 5) (width 0.25) (layer "F.Cu") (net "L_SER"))
 (segment (start 3 3) (end 5.5375 3) (width 0.25) (layer "F.Cu") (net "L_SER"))
 (segment (start 39.5 17.365) (end 39.5 13.555) (width 0.25) (layer "F.Cu") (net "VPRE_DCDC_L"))
 (segment (start 37.875 17.365) (end 39.5 17.365) (width 0.25) (layer "F.Cu") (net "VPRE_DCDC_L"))
 (segment (start 40.225 13.555) (end 40.225 13.5) (width 0.25) (layer "F.Cu") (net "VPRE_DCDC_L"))
 (segment (start 37.875 13.555) (end 40.225 13.555) (width 0.25) (layer "F.Cu") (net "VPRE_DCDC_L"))
 (segment (start 28.125 16.094999) (end 26.3 16.094999) (width 0.25) (layer "F.Cu") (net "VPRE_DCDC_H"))
 (segment (start 25.475 14) (end 25.475 16.5) (width 0.25) (layer "F.Cu") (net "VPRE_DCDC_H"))
 (segment (start 28.125 13.555) (end 26.3 13.555) (width 0.25) (layer "F.Cu") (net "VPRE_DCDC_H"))
 (segment (start 26.3 16.094999) (end 25.475 16.5) (width 0.25) (layer "F.Cu") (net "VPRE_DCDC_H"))
 (segment (start 26.3 13.555) (end 25.475 14) (width 0.25) (layer "F.Cu") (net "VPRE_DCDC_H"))
 (segment (start 26.5 18.635) (end 24.775 18.635) (width 0.25) (layer "F.Cu") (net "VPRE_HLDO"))
 (segment (start 28.125 18.635) (end 26.5 18.635) (width 0.25) (layer "F.Cu") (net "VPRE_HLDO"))
 (segment (start 24.775 21.5) (end 24.775 24) (width 0.25) (layer "F.Cu") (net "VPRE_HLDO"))
 (segment (start 24.775 18.635) (end 24.775 21.5) (width 0.25) (layer "F.Cu") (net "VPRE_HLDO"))
 (segment (start 22.5375 10) (end 19.4625 10) (width 0.25) (layer "F.Cu") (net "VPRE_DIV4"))
 (segment (start 16.5375 10) (end 13.4625 10) (width 0.25) (layer "F.Cu") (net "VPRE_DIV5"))
 (segment (start 10.5375 10) (end 7.4625 10) (width 0.25) (layer "F.Cu") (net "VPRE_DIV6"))
 (segment (start 37.875 19.905) (end 39 19.905) (width 0.25) (layer "F.Cu") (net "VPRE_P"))
 (via (at 39 19.905) (size 0.6) (drill 0.3) (layers "F.Cu" "B.Cu") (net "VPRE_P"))
 (segment (start 47 15) (end 53 15) (width 0.25) (layer "B.Cu") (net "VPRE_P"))
 (segment (start 39 19.905) (end 47 19.905) (width 0.25) (layer "B.Cu") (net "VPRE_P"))
 (segment (start 47 19.905) (end 47 15) (width 0.25) (layer "B.Cu") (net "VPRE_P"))
 (segment (start 37.875 21.175) (end 39 21.175) (width 0.25) (layer "F.Cu") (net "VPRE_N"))
 (via (at 39 21.175) (size 0.6) (drill 0.3) (layers "F.Cu" "B.Cu") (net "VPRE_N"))
 (segment (start 48 17.5) (end 53 17.5) (width 0.25) (layer "B.Cu") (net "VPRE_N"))
 (segment (start 48 21.175) (end 48 17.5) (width 0.25) (layer "B.Cu") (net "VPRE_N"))
 (segment (start 39 21.175) (end 48 21.175) (width 0.25) (layer "B.Cu") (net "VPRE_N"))
 (segment (start 49 27) (end 49 20) (width 0.25) (layer "F.Cu") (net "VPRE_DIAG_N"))
 (segment (start 49 20) (end 53 20) (width 0.25) (layer "F.Cu") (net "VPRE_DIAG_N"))
 (segment (start 46 27) (end 44.825 27) (width 0.25) (layer "F.Cu") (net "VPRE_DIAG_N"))
 (segment (start 37.875 16.094999) (end 38.7 16.094999) (width 0.25) (layer "F.Cu") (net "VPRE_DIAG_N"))
 (segment (start 44.825 27) (end 49 27) (width 0.25) (layer "F.Cu") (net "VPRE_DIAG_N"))
 (segment (start 46 16.094999) (end 46 27) (width 0.25) (layer "F.Cu") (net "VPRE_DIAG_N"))
 (via (at 46 16.094999) (size 0.6) (drill 0.3) (layers "F.Cu" "B.Cu") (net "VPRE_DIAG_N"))
 (via (at 38.7 16.094999) (size 0.6) (drill 0.3) (layers "F.Cu" "B.Cu") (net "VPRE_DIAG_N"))
 (segment (start 38.7 16.094999) (end 46 16.094999) (width 0.25) (layer "B.Cu") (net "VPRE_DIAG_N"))
 (segment (start 8.4625 5) (end 10.5375 5) (width 0.25) (layer "F.Cu") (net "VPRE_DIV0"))
 (segment (start 13.4625 5) (end 16.5375 5) (width 0.25) (layer "F.Cu") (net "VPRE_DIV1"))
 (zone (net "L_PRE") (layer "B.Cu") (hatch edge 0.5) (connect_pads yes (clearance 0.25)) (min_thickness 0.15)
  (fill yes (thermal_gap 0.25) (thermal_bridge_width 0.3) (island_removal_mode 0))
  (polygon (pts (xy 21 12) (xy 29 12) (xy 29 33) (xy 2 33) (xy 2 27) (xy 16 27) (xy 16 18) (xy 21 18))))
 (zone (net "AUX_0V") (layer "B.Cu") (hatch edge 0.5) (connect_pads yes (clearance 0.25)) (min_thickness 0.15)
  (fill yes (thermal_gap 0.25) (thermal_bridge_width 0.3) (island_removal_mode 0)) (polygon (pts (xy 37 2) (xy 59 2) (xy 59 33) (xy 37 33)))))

